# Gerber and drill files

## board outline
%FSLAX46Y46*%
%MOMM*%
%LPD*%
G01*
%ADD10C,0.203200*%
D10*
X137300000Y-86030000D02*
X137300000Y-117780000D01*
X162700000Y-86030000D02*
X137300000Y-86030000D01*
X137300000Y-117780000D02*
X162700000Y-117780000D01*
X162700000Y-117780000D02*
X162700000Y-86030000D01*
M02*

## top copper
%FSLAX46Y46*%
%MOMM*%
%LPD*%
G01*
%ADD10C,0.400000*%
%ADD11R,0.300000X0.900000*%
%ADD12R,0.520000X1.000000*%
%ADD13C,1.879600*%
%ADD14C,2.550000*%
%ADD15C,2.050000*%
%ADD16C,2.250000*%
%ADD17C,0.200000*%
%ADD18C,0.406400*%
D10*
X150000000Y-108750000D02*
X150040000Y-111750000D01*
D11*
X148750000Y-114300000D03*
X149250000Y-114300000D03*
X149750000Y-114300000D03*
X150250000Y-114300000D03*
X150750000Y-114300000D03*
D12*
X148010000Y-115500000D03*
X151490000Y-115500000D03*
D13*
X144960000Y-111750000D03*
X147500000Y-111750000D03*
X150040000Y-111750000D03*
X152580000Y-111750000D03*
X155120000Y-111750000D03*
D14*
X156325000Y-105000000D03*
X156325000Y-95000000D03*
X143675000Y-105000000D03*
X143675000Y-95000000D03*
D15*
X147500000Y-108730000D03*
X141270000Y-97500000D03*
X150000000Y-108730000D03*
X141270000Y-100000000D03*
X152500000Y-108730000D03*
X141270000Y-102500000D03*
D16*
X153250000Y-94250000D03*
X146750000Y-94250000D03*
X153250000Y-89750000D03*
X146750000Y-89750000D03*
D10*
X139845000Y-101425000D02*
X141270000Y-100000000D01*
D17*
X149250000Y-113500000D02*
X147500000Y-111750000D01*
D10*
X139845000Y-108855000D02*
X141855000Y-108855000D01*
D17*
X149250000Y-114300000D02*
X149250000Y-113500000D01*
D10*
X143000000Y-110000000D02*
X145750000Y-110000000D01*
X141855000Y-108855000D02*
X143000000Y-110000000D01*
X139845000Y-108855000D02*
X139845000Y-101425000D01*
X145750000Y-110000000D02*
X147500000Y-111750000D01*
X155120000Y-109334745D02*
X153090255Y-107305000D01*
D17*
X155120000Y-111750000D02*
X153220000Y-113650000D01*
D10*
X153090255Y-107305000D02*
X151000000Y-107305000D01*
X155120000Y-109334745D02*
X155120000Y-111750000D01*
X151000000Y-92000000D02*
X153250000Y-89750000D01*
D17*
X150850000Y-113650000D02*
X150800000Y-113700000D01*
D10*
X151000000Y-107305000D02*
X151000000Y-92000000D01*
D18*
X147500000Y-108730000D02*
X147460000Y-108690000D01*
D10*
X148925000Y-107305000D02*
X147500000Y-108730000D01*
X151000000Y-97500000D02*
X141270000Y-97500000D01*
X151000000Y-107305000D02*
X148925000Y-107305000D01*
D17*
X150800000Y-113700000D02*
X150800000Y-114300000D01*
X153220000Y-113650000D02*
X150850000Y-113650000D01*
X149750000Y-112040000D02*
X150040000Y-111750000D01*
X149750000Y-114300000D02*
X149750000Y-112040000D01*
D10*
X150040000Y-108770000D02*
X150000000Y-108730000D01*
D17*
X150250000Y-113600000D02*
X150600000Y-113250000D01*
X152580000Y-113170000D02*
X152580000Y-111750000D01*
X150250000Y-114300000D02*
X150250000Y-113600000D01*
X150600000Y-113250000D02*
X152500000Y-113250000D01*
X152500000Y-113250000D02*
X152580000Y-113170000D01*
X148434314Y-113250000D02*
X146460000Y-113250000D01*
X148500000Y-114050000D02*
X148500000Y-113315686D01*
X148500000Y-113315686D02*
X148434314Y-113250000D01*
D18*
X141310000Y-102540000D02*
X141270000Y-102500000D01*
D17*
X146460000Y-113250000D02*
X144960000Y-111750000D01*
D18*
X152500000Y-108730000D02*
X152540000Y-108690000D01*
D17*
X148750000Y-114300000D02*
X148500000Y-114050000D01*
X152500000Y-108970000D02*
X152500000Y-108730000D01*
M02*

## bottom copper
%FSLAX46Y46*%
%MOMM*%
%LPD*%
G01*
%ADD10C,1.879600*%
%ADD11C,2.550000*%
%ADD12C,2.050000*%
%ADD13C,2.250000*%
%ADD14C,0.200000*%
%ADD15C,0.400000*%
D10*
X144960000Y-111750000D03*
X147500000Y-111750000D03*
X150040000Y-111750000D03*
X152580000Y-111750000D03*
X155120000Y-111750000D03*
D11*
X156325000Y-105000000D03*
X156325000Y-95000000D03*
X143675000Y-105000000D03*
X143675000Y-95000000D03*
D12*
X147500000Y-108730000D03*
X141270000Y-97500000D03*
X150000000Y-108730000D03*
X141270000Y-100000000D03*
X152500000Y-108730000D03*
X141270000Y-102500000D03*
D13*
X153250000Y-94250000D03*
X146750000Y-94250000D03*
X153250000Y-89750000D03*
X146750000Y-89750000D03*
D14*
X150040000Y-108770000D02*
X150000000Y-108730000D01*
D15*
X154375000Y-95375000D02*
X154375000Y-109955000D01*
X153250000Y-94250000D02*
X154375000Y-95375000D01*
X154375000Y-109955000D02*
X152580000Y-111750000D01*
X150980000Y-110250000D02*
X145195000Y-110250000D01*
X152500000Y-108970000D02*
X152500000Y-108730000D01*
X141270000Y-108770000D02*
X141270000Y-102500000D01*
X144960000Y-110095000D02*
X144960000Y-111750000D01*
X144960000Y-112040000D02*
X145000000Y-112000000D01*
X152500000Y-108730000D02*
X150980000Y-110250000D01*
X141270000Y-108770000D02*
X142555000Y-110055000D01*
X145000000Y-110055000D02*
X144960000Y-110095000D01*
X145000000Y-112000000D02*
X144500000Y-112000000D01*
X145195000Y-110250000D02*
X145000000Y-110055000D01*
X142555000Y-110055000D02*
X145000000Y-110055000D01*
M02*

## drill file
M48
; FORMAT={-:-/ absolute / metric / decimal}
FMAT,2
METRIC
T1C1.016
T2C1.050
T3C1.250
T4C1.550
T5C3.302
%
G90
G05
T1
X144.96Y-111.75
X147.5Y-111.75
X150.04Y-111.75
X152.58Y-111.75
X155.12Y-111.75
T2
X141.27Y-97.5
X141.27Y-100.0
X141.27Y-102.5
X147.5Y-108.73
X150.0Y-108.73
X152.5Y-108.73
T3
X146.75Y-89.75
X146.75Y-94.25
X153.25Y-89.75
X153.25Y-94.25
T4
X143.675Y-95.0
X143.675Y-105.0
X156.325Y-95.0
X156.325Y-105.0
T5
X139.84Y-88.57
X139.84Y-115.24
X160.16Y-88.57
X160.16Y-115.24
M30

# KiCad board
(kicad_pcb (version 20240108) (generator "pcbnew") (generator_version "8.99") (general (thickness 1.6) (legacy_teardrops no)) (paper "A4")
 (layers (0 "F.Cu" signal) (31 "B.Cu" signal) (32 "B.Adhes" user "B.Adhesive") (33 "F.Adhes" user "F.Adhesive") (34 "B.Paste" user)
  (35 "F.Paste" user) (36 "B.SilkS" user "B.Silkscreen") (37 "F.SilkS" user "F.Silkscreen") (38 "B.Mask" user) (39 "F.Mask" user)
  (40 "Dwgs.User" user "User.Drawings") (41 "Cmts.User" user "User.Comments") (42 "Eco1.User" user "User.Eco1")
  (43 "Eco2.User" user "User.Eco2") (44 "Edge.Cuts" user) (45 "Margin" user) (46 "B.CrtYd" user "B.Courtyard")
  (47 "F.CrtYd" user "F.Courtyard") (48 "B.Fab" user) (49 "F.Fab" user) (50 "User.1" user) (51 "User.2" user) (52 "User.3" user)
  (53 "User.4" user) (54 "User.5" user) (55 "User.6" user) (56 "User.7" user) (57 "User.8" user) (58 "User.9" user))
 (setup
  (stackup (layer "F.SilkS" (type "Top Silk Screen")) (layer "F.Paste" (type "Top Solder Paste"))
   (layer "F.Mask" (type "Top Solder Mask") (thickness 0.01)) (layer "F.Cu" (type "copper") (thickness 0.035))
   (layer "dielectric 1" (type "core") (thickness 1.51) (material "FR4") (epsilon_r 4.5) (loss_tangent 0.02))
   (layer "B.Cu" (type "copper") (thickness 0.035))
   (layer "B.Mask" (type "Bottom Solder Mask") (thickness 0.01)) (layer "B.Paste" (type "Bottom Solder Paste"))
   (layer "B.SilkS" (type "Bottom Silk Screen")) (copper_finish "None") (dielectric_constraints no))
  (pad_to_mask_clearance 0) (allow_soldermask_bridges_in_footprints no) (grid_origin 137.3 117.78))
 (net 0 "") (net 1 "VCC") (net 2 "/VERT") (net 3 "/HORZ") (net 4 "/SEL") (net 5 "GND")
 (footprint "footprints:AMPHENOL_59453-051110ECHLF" (layer "F.Cu") (at 149.75 115.5)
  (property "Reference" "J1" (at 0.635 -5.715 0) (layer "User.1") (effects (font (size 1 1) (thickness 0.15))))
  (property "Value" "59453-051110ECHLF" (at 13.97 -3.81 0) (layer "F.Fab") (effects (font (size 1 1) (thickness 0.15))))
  (pad "1" smd rect (at -1 -1.2) (size 0.3 0.9) (layers "F.Cu" "F.Paste" "F.Mask") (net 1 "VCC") (solder_mask_margin 0.102))
  (pad "2" smd rect (at -0.5 -1.2) (size 0.3 0.9) (layers "F.Cu" "F.Paste" "F.Mask") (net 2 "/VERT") (solder_mask_margin 0.102))
  (pad "3" smd rect (at 0 -1.2) (size 0.3 0.9) (layers "F.Cu" "F.Paste" "F.Mask") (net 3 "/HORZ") (solder_mask_margin 0.102))
  (pad "4" smd rect (at 0.5 -1.2) (size 0.3 0.9) (layers "F.Cu" "F.Paste" "F.Mask") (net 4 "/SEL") (solder_mask_margin 0.102))
  (pad "5" smd rect (at 1 -1.2) (size 0.3 0.9) (layers "F.Cu" "F.Paste" "F.Mask") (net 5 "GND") (solder_mask_margin 0.102))
  (pad "S1" smd rect (at -1.74 0) (size 0.52 1) (layers "F.Cu" "F.Paste" "F.Mask") (solder_mask_margin 0.102))
  (pad "S2" smd rect (at 1.74 0) (size 0.52 1) (layers "F.Cu" "F.Paste" "F.Mask") (solder_mask_margin 0.102)))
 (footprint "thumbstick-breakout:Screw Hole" (layer "F.Cu") (at 139.84 115.24)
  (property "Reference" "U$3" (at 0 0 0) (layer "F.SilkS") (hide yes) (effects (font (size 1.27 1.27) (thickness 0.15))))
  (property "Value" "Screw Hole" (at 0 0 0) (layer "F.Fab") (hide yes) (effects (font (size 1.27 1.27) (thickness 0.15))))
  (pad "" np_thru_hole circle (at 0 0) (size 3.302 3.302) (drill 3.302) (layers "F&B.Cu" "*.Mask")))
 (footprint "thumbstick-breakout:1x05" (layer "F.Cu") (at 150.04 111.75)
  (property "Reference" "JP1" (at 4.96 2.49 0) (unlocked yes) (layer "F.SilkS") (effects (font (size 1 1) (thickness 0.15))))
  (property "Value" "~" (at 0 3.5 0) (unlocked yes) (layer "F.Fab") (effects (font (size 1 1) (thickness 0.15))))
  (pad "1" thru_hole circle (at -5.08 0 270) (size 1.8796 1.8796) (drill 1.016) (layers "*.Cu" "*.Mask") (remove_unused_layers no)
   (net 1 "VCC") (solder_mask_margin 0.1) (thermal_bridge_angle 0))
  (pad "2" thru_hole circle (at -2.54 0 270) (size 1.8796 1.8796) (drill 1.016) (layers "*.Cu" "*.Mask") (remove_unused_layers no)
   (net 2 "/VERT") (solder_mask_margin 0.1) (thermal_bridge_angle 0))
  (pad "3" thru_hole circle (at 0 0 270) (size 1.8796 1.8796) (drill 1.016) (layers "*.Cu" "*.Mask") (remove_unused_layers no)
   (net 3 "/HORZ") (solder_mask_margin 0.1) (thermal_bridge_angle 0))
  (pad "4" thru_hole circle (at 2.54 0 270) (size 1.8796 1.8796) (drill 1.016) (layers "*.Cu" "*.Mask") (remove_unused_layers no)
   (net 4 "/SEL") (solder_mask_margin 0.1) (thermal_bridge_angle 0))
  (pad "5" thru_hole circle (at 5.08 0 270) (size 1.8796 1.8796) (drill 1.016) (layers "*.Cu" "*.Mask") (remove_unused_layers no)
   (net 5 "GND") (solder_mask_margin 0.1) (thermal_bridge_angle 0)))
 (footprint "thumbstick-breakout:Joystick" (layer "F.Cu") (at 150 100 180)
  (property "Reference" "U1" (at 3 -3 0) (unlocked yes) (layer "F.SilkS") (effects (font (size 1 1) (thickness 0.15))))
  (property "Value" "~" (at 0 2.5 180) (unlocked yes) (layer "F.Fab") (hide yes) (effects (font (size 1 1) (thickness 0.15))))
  (pad "" thru_hole circle (at -6.325 -5 180) (size 2.55 2.55) (drill 1.55) (layers "*.Cu" "*.Mask") (remove_unused_layers no)
   (solder_mask_margin 0.1))
  (pad "" thru_hole circle (at -6.325 5 180) (size 2.55 2.55) (drill 1.55) (layers "*.Cu" "*.Mask") (remove_unused_layers no)
   (solder_mask_margin 0.1))
  (pad "" thru_hole circle (at 6.325 -5 180) (size 2.55 2.55) (drill 1.55) (layers "*.Cu" "*.Mask") (remove_unused_layers no)
   (solder_mask_margin 0.1))
  (pad "" thru_hole circle (at 6.325 5 180) (size 2.55 2.55) (drill 1.55) (layers "*.Cu" "*.Mask") (remove_unused_layers no)
   (solder_mask_margin 0.1))
  (pad "1" thru_hole circle (at 2.5 -8.73 180) (size 2.05 2.05) (drill 1.05) (layers "*.Cu" "*.Mask") (remove_unused_layers no)
   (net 5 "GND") (solder_mask_margin 0.1))
  (pad "1'" thru_hole circle (at 8.73 2.5 180) (size 2.05 2.05) (drill 1.05) (layers "*.Cu" "*.Mask") (remove_unused_layers no)
   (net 5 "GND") (solder_mask_margin 0.1))
  (pad "2" thru_hole circle (at 0 -8.73 180) (size 2.05 2.05) (drill 1.05) (layers "*.Cu" "*.Mask") (remove_unused_layers no)
   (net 3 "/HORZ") (solder_mask_margin 0.1))
  (pad "2'" thru_hole circle (at 8.73 0 180) (size 2.05 2.05) (drill 1.05) (layers "*.Cu" "*.Mask") (remove_unused_layers no)
   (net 2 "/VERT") (solder_mask_margin 0.1))
  (pad "3" thru_hole circle (at -2.5 -8.73 180) (size 2.05 2.05) (drill 1.05) (layers "*.Cu" "*.Mask") (remove_unused_layers no)
   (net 1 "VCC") (solder_mask_margin 0.1))
  (pad "3'" thru_hole circle (at 8.73 -2.5 180) (size 2.05 2.05) (drill 1.05) (layers "*.Cu" "*.Mask") (remove_unused_layers no)
   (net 1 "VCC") (solder_mask_margin 0.1))
  (pad "a" thru_hole circle (at -3.25 5.75 180) (size 2.25 2.25) (drill 1.25) (layers "*.Cu" "*.Mask") (remove_unused_layers no)
   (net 4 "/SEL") (solder_mask_margin 0.1))
  (pad "b" thru_hole circle (at 3.25 5.75 180) (size 2.25 2.25) (drill 1.25) (layers "*.Cu" "*.Mask") (remove_unused_layers no)
   (solder_mask_margin 0.1))
  (pad "c" thru_hole circle (at -3.25 10.25 180) (size 2.25 2.25) (drill 1.25) (layers "*.Cu" "*.Mask") (remove_unused_layers no)
   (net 5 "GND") (solder_mask_margin 0.1))
  (pad "d" thru_hole circle (at 3.25 10.25 180) (size 2.25 2.25) (drill 1.25) (layers "*.Cu" "*.Mask") (remove_unused_layers no)
   (solder_mask_margin 0.1)))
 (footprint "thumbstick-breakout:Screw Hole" (layer "F.Cu") (at 160.16 115.24)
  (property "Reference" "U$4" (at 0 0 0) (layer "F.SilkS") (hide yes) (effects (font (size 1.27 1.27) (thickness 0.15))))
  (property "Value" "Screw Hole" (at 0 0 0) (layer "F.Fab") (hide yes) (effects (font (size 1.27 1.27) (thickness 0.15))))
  (pad "" np_thru_hole circle (at 0 0) (size 3.302 3.302) (drill 3.302) (layers "F&B.Cu" "*.Mask")))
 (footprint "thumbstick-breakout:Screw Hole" (layer "F.Cu") (at 160.16 88.57)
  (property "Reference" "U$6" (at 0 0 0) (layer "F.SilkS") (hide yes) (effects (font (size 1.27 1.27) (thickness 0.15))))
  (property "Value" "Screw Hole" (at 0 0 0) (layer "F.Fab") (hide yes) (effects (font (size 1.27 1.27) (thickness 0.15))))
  (pad "" np_thru_hole circle (at 0 0) (size 3.302 3.302) (drill 3.302) (layers "F&B.Cu" "*.Mask")))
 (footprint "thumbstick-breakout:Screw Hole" (layer "F.Cu") (at 139.84 88.57)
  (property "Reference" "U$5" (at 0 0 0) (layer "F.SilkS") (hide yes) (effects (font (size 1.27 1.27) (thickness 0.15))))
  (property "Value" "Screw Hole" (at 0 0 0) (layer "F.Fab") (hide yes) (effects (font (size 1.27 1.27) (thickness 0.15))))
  (pad "" np_thru_hole circle (at 0 0) (size 3.302 3.302) (drill 3.302) (layers "F&B.Cu" "*.Mask")))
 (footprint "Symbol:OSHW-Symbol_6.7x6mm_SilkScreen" (layer "B.Cu") (at 150 99.685893 180)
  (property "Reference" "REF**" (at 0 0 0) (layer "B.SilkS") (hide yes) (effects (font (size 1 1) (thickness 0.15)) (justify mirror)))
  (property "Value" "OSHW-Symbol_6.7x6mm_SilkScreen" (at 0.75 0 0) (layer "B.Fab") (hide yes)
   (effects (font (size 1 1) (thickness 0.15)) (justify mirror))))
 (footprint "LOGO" (layer "B.Cu") (at 157.5 87.5 180)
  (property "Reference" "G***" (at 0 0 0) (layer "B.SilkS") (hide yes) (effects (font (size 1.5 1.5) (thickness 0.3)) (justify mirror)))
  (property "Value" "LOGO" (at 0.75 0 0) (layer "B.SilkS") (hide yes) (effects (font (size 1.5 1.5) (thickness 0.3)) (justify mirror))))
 (gr_line (start 150 108.75) (end 150.04 111.75) (stroke (width 0.4) (type default)) (layer "F.Cu") (net 3))
 (gr_line (start 137.3 86.03) (end 137.3 117.78) (stroke (width 0.2032) (type solid)) (layer "Edge.Cuts"))
 (gr_line (start 162.7 86.03) (end 137.3 86.03) (stroke (width 0.2032) (type solid)) (layer "Edge.Cuts"))
 (gr_line (start 137.3 117.78) (end 162.7 117.78) (stroke (width 0.2032) (type solid)) (layer "Edge.Cuts"))
 (gr_line (start 162.7 117.78) (end 162.7 86.03) (stroke (width 0.2032) (type solid)) (layer "Edge.Cuts"))
 (segment (start 139.845 101.425) (end 141.27 100) (width 0.4) (layer "F.Cu") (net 2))
 (segment (start 149.25 113.5) (end 147.5 111.75) (width 0.2) (layer "F.Cu") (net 2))
 (segment (start 139.845 108.855) (end 141.855 108.855) (width 0.4) (layer "F.Cu") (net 2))
 (segment (start 149.25 114.3) (end 149.25 113.5) (width 0.2) (layer "F.Cu") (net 2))
 (segment (start 143 110) (end 145.75 110) (width 0.4) (layer "F.Cu") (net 2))
 (segment (start 141.855 108.855) (end 143 110) (width 0.4) (layer "F.Cu") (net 2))
 (segment (start 139.845 108.855) (end 139.845 101.425) (width 0.4) (layer "F.Cu") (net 2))
 (segment (start 145.75 110) (end 147.5 111.75) (width 0.4) (layer "F.Cu") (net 2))
 (segment (start 155.12 109.334745) (end 153.090255 107.305) (width 0.4) (layer "F.Cu") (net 5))
 (segment (start 155.12 111.75) (end 153.22 113.65) (width 0.2) (layer "F.Cu") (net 5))
 (segment (start 153.090255 107.305) (end 151 107.305) (width 0.4) (layer "F.Cu") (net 5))
 (segment (start 155.12 109.334745) (end 155.12 111.75) (width 0.4) (layer "F.Cu") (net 5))
 (segment (start 151 92) (end 153.25 89.75) (width 0.4) (layer "F.Cu") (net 5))
 (segment (start 150.85 113.65) (end 150.8 113.7) (width 0.2) (layer "F.Cu") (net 5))
 (segment (start 151 107.305) (end 151 92) (width 0.4) (layer "F.Cu") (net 5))
 (segment (start 147.5 108.73) (end 147.46 108.69) (width 0.4064) (layer "F.Cu") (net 5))
 (segment (start 148.925 107.305) (end 147.5 108.73) (width 0.4) (layer "F.Cu") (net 5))
 (segment (start 151 97.5) (end 141.27 97.5) (width 0.4) (layer "F.Cu") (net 5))
 (segment (start 151 107.305) (end 148.925 107.305) (width 0.4) (layer "F.Cu") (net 5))
 (segment (start 150.8 113.7) (end 150.8 114.3) (width 0.2) (layer "F.Cu") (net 5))
 (segment (start 153.22 113.65) (end 150.85 113.65) (width 0.2) (layer "F.Cu") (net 5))
 (segment (start 149.75 112.04) (end 150.04 111.75) (width 0.2) (layer "F.Cu") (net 3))
 (segment (start 149.75 114.3) (end 149.75 112.04) (width 0.2) (layer "F.Cu") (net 3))
 (segment (start 150.04 108.77) (end 150 108.73) (width 0.4) (layer "F.Cu") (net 3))
 (segment (start 150.04 108.77) (end 150 108.73) (width 0.2) (layer "B.Cu") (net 3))
 (segment (start 150.25 113.6) (end 150.6 113.25) (width 0.2) (layer "F.Cu") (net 4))
 (segment (start 152.58 113.17) (end 152.58 111.75) (width 0.2) (layer "F.Cu") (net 4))
 (segment (start 150.25 114.3) (end 150.25 113.6) (width 0.2) (layer "F.Cu") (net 4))
 (segment (start 150.6 113.25) (end 152.5 113.25) (width 0.2) (layer "F.Cu") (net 4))
 (segment (start 152.5 113.25) (end 152.58 113.17) (width 0.2) (layer "F.Cu") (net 4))
 (segment (start 154.375 95.375) (end 154.375 109.955) (width 0.4) (layer "B.Cu") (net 4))
 (segment (start 153.25 94.25) (end 154.375 95.375) (width 0.4) (layer "B.Cu") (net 4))
 (segment (start 154.375 109.955) (end 152.58 111.75) (width 0.4) (layer "B.Cu") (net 4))
 (segment (start 148.434314 113.25) (end 146.46 113.25) (width 0.2) (layer "F.Cu") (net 1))
 (segment (start 148.5 114.05) (end 148.5 113.315686) (width 0.2) (layer "F.Cu") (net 1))
 (segment (start 148.5 113.315686) (end 148.434314 113.25) (width 0.2) (layer "F.Cu") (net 1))
 (segment (start 141.31 102.54) (end 141.27 102.5) (width 0.4064) (layer "F.Cu") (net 1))
 (segment (start 146.46 113.25) (end 144.96 111.75) (width 0.2) (layer "F.Cu") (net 1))
 (segment (start 152.5 108.73) (end 152.54 108.69) (width 0.4064) (layer "F.Cu") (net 1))
 (segment (start 148.75 114.3) (end 148.5 114.05) (width 0.2) (layer "F.Cu") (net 1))
 (segment (start 152.5 108.97) (end 152.5 108.73) (width 0.2) (layer "F.Cu") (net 1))
 (segment (start 150.98 110.25) (end 145.195 110.25) (width 0.4) (layer "B.Cu") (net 1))
 (segment (start 152.5 108.97) (end 152.5 108.73) (width 0.4) (layer "B.Cu") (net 1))
 (segment (start 141.27 108.77) (end 141.27 102.5) (width 0.4) (layer "B.Cu") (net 1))
 (segment (start 144.96 110.095) (end 144.96 111.75) (width 0.4) (layer "B.Cu") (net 1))
 (segment (start 144.96 112.04) (end 145 112) (width 0.4) (layer "B.Cu") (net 1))
 (segment (start 152.5 108.73) (end 150.98 110.25) (width 0.4) (layer "B.Cu") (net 1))
 (segment (start 141.27 108.77) (end 142.555 110.055) (width 0.4) (layer "B.Cu") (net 1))
 (segment (start 145 110.055) (end 144.96 110.095) (width 0.4) (layer "B.Cu") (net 1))
 (segment (start 145 112) (end 144.5 112) (width 0.4) (layer "B.Cu") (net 1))
 (segment (start 145.195 110.25) (end 145 110.055) (width 0.4) (layer "B.Cu") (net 1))
 (segment (start 142.555 110.055) (end 145 110.055) (width 0.4) (layer "B.Cu") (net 1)))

